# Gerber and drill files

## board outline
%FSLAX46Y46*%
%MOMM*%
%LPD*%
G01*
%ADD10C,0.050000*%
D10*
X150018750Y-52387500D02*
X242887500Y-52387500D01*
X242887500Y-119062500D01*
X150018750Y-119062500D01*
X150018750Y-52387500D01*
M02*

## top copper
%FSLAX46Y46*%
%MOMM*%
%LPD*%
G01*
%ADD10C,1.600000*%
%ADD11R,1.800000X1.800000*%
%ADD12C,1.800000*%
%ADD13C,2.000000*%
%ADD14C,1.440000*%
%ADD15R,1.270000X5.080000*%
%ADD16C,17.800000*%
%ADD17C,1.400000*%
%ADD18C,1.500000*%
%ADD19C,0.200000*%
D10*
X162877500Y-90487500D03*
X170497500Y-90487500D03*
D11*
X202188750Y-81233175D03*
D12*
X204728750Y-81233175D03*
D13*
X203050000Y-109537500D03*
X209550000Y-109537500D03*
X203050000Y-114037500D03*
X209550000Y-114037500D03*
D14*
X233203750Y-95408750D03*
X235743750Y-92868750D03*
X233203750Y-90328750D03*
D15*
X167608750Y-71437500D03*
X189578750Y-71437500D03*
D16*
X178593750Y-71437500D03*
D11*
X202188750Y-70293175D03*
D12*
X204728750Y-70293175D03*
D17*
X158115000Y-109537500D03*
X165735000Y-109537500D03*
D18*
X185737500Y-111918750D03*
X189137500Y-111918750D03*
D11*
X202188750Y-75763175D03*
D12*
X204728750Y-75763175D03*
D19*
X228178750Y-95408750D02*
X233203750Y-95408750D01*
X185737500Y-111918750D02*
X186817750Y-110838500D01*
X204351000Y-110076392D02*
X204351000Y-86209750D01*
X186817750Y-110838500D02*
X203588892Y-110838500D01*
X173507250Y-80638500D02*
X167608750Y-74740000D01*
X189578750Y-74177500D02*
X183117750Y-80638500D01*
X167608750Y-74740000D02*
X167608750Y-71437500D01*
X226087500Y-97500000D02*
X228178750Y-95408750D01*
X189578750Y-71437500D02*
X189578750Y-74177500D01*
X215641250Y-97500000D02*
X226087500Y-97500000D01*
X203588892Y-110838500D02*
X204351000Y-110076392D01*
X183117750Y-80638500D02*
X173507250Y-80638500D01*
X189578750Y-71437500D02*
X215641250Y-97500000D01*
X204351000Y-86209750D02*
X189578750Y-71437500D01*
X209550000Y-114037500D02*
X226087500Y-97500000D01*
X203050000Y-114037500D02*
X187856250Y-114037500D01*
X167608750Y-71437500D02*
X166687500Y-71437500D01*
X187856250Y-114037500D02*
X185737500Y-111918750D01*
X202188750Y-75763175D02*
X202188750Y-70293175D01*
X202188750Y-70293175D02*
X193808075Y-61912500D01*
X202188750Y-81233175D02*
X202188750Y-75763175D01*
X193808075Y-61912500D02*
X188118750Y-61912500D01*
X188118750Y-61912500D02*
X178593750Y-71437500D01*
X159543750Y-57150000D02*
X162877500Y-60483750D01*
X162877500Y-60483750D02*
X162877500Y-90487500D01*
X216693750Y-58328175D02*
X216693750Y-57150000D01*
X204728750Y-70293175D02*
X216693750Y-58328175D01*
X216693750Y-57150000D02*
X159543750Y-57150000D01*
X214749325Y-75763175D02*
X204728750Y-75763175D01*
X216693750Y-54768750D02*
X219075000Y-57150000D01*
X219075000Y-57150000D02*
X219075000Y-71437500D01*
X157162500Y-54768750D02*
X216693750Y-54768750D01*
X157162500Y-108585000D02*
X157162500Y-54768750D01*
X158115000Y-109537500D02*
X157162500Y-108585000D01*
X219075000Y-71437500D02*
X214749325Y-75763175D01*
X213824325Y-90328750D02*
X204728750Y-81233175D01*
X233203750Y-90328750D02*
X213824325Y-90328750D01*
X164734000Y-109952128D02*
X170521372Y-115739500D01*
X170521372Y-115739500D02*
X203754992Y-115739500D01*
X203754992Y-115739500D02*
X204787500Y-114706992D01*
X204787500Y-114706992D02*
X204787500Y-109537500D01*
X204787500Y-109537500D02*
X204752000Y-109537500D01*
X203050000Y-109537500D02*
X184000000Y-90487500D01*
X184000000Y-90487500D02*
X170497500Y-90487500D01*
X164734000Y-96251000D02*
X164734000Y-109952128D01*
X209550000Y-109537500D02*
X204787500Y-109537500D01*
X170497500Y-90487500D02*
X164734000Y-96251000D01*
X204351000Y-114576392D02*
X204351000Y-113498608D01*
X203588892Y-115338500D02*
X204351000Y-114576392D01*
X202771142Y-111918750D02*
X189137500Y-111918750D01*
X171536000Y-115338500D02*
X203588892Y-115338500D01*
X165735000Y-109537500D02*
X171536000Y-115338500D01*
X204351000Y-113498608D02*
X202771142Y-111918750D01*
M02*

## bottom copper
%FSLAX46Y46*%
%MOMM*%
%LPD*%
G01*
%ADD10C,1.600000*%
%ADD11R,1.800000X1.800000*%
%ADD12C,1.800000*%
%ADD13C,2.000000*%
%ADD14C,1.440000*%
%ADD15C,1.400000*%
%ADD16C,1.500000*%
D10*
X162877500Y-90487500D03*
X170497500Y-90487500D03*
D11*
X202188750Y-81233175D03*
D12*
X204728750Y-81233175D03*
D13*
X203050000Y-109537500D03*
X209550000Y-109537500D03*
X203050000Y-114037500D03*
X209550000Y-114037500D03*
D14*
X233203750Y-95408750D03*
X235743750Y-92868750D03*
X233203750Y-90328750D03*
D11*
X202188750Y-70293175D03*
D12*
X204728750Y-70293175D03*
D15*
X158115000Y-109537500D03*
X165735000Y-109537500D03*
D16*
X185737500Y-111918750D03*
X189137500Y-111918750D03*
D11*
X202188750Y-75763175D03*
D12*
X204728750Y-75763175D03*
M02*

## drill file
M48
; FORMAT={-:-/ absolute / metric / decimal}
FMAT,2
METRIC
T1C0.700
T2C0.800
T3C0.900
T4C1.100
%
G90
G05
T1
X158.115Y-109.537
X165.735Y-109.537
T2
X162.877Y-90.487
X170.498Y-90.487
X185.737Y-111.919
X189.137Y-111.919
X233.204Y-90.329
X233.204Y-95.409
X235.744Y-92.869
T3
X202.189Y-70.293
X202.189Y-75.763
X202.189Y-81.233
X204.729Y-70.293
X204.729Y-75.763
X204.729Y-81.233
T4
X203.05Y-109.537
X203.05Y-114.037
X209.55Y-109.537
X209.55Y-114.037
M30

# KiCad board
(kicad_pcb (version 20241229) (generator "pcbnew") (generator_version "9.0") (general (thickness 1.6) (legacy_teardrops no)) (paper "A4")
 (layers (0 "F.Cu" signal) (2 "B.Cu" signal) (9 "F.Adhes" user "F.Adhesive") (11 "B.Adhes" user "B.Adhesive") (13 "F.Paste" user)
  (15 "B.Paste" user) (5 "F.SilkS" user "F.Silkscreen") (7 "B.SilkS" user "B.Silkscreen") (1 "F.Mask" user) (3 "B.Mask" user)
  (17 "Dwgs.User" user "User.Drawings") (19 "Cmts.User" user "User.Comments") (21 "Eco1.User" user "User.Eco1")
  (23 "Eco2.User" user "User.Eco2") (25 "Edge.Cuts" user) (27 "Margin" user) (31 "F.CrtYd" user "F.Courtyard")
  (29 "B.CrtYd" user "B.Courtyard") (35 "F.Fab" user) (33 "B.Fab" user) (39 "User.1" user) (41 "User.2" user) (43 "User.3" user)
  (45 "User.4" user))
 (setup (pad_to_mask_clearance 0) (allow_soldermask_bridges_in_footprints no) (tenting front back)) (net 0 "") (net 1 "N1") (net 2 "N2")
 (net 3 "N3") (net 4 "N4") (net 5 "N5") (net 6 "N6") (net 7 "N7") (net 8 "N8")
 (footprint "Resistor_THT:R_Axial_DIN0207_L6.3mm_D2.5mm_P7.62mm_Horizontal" (layer "F.Cu") (at 162.8775 90.4875)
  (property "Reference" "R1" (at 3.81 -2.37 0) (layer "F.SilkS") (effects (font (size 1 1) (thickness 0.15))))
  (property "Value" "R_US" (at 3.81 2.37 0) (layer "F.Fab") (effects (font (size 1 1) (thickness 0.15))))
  (pad "1" thru_hole circle (at 0 0) (size 1.6 1.6) (drill 0.8) (layers "*.Cu" "*.Mask") (remove_unused_layers no) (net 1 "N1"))
  (pad "2" thru_hole circle (at 7.62 0) (size 1.6 1.6) (drill 0.8) (layers "*.Cu" "*.Mask") (remove_unused_layers no) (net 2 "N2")))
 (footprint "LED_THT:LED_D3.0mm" (layer "F.Cu") (at 202.18875 81.233175)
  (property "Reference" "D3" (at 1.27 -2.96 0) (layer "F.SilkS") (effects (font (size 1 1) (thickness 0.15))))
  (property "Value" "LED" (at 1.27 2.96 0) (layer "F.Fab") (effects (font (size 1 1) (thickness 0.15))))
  (pad "1" thru_hole rect (at 0 0) (size 1.8 1.8) (drill 0.9) (layers "*.Cu" "*.Mask") (remove_unused_layers no) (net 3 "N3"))
  (pad "2" thru_hole circle (at 2.54 0) (size 1.8 1.8) (drill 0.9) (layers "*.Cu" "*.Mask") (remove_unused_layers no) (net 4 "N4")))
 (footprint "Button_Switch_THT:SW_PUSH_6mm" (layer "F.Cu") (at 203.05 109.5375)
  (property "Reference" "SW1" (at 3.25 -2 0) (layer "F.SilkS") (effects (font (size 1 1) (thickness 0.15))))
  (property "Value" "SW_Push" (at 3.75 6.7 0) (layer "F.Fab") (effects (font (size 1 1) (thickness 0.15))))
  (pad "1" thru_hole circle (at 0 0 90) (size 2 2) (drill 1.1) (layers "*.Cu" "*.Mask") (remove_unused_layers no) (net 2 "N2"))
  (pad "1" thru_hole circle (at 6.5 0 90) (size 2 2) (drill 1.1) (layers "*.Cu" "*.Mask") (remove_unused_layers no) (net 2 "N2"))
  (pad "2" thru_hole circle (at 0 4.5 90) (size 2 2) (drill 1.1) (layers "*.Cu" "*.Mask") (remove_unused_layers no) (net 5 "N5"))
  (pad "2" thru_hole circle (at 6.5 4.5 90) (size 2 2) (drill 1.1) (layers "*.Cu" "*.Mask") (remove_unused_layers no) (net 5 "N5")))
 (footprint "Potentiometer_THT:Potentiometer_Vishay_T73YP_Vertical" (layer "F.Cu") (at 233.20375 95.40875)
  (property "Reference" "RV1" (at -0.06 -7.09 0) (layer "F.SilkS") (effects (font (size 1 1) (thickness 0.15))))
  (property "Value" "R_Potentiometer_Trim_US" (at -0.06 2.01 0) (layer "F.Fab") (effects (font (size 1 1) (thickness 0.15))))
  (pad "1" thru_hole circle (at 0 0) (size 1.44 1.44) (drill 0.8) (layers "*.Cu" "*.Mask") (remove_unused_layers no) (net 5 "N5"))
  (pad "2" thru_hole circle (at 2.54 -2.54) (size 1.44 1.44) (drill 0.8) (layers "*.Cu" "*.Mask") (remove_unused_layers no) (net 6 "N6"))
  (pad "3" thru_hole circle (at 0 -5.08) (size 1.44 1.44) (drill 0.8) (layers "*.Cu" "*.Mask") (remove_unused_layers no) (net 4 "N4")))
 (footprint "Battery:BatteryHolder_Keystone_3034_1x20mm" (layer "F.Cu") (at 178.59375 71.4375)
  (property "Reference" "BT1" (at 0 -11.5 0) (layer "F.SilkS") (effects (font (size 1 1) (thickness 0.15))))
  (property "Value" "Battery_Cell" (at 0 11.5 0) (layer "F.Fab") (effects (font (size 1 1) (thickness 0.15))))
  (pad "1" smd rect (at -10.985 0) (size 1.27 5.08) (layers "F.Cu" "F.Mask" "F.Paste") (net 5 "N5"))
  (pad "1" smd rect (at 10.985 0) (size 1.27 5.08) (layers "F.Cu" "F.Mask" "F.Paste") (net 5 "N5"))
  (pad "2" smd circle (at 0 0) (size 17.8 17.8) (layers "F.Cu" "F.Mask") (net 3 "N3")))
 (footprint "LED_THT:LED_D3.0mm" (layer "F.Cu") (at 202.18875 70.293175)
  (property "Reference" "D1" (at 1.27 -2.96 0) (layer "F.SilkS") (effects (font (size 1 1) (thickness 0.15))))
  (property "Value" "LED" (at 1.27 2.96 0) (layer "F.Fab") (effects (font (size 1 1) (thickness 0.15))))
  (pad "1" thru_hole rect (at 0 0) (size 1.8 1.8) (drill 0.9) (layers "*.Cu" "*.Mask") (remove_unused_layers no) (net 3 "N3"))
  (pad "2" thru_hole circle (at 2.54 0) (size 1.8 1.8) (drill 0.9) (layers "*.Cu" "*.Mask") (remove_unused_layers no) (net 1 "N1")))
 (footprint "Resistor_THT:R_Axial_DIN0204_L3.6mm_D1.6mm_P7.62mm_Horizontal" (layer "F.Cu") (at 158.115 109.5375)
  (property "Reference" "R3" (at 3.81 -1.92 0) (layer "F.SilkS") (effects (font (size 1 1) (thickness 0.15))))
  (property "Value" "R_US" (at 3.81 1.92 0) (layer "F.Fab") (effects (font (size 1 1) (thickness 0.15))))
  (pad "1" thru_hole circle (at 0 0) (size 1.4 1.4) (drill 0.7) (layers "*.Cu" "*.Mask") (remove_unused_layers no) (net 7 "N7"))
  (pad "2" thru_hole circle (at 7.62 0) (size 1.4 1.4) (drill 0.7) (layers "*.Cu" "*.Mask") (remove_unused_layers no) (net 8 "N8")))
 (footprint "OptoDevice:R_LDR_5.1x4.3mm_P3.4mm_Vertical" (layer "F.Cu") (at 185.7375 111.91875)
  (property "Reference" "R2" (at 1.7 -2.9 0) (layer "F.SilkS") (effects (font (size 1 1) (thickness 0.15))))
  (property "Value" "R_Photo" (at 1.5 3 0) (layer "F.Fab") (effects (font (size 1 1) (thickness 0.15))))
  (pad "1" thru_hole circle (at 0 0) (size 1.5 1.5) (drill 0.8) (layers "*.Cu" "*.Mask") (remove_unused_layers no) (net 5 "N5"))
  (pad "2" thru_hole circle (at 3.4 0) (size 1.5 1.5) (drill 0.8) (layers "*.Cu" "*.Mask") (remove_unused_layers no) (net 8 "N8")))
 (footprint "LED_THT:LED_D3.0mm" (layer "F.Cu") (at 202.18875 75.763175)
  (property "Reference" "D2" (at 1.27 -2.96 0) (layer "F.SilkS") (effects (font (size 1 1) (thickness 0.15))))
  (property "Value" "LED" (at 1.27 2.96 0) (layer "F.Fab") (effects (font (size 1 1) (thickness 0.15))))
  (pad "1" thru_hole rect (at 0 0) (size 1.8 1.8) (drill 0.9) (layers "*.Cu" "*.Mask") (remove_unused_layers no) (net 3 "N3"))
  (pad "2" thru_hole circle (at 2.54 0) (size 1.8 1.8) (drill 0.9) (layers "*.Cu" "*.Mask") (remove_unused_layers no) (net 7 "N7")))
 (gr_rect (start 150.01875 52.3875) (end 242.8875 119.0625) (stroke (width 0.05) (type default)) (fill no) (layer "Edge.Cuts"))
 (segment (start 228.17875 95.40875) (end 233.20375 95.40875) (width 0.2) (layer "F.Cu") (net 5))
 (segment (start 185.7375 111.91875) (end 186.81775 110.8385) (width 0.2) (layer "F.Cu") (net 5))
 (segment (start 204.351 110.076392) (end 204.351 86.20975) (width 0.2) (layer "F.Cu") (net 5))
 (segment (start 186.81775 110.8385) (end 203.588892 110.8385) (width 0.2) (layer "F.Cu") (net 5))
 (segment (start 173.50725 80.6385) (end 167.60875 74.74) (width 0.2) (layer "F.Cu") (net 5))
 (segment (start 189.57875 74.1775) (end 183.11775 80.6385) (width 0.2) (layer "F.Cu") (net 5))
 (segment (start 167.60875 74.74) (end 167.60875 71.4375) (width 0.2) (layer "F.Cu") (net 5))
 (segment (start 226.0875 97.5) (end 228.17875 95.40875) (width 0.2) (layer "F.Cu") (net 5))
 (segment (start 189.57875 71.4375) (end 189.57875 74.1775) (width 0.2) (layer "F.Cu") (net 5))
 (segment (start 215.64125 97.5) (end 226.0875 97.5) (width 0.2) (layer "F.Cu") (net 5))
 (segment (start 203.588892 110.8385) (end 204.351 110.076392) (width 0.2) (layer "F.Cu") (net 5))
 (segment (start 183.11775 80.6385) (end 173.50725 80.6385) (width 0.2) (layer "F.Cu") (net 5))
 (segment (start 189.57875 71.4375) (end 215.64125 97.5) (width 0.2) (layer "F.Cu") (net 5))
 (segment (start 204.351 86.20975) (end 189.57875 71.4375) (width 0.2) (layer "F.Cu") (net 5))
 (segment (start 209.55 114.0375) (end 226.0875 97.5) (width 0.2) (layer "F.Cu") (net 5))
 (segment (start 203.05 114.0375) (end 187.85625 114.0375) (width 0.2) (layer "F.Cu") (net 5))
 (segment (start 167.60875 71.4375) (end 166.6875 71.4375) (width 0.2) (layer "F.Cu") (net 5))
 (segment (start 187.85625 114.0375) (end 185.7375 111.91875) (width 0.2) (layer "F.Cu") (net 5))
 (segment (start 202.18875 75.763175) (end 202.18875 70.293175) (width 0.2) (layer "F.Cu") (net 3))
 (segment (start 202.18875 70.293175) (end 193.808075 61.9125) (width 0.2) (layer "F.Cu") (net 3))
 (segment (start 202.18875 81.233175) (end 202.18875 75.763175) (width 0.2) (layer "F.Cu") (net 3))
 (segment (start 193.808075 61.9125) (end 188.11875 61.9125) (width 0.2) (layer "F.Cu") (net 3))
 (segment (start 188.11875 61.9125) (end 178.59375 71.4375) (width 0.2) (layer "F.Cu") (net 3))
 (segment (start 159.54375 57.15) (end 162.8775 60.48375) (width 0.2) (layer "F.Cu") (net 1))
 (segment (start 162.8775 60.48375) (end 162.8775 90.4875) (width 0.2) (layer "F.Cu") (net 1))
 (segment (start 216.69375 58.328175) (end 216.69375 57.15) (width 0.2) (layer "F.Cu") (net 1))
 (segment (start 204.72875 70.293175) (end 216.69375 58.328175) (width 0.2) (layer "F.Cu") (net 1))
 (segment (start 216.69375 57.15) (end 159.54375 57.15) (width 0.2) (layer "F.Cu") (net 1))
 (segment (start 214.749325 75.763175) (end 204.72875 75.763175) (width 0.2) (layer "F.Cu") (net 7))
 (segment (start 216.69375 54.76875) (end 219.075 57.15) (width 0.2) (layer "F.Cu") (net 7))
 (segment (start 219.075 57.15) (end 219.075 71.4375) (width 0.2) (layer "F.Cu") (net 7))
 (segment (start 157.1625 54.76875) (end 216.69375 54.76875) (width 0.2) (layer "F.Cu") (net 7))
 (segment (start 157.1625 108.585) (end 157.1625 54.76875) (width 0.2) (layer "F.Cu") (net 7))
 (segment (start 158.115 109.5375) (end 157.1625 108.585) (width 0.2) (layer "F.Cu") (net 7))
 (segment (start 219.075 71.4375) (end 214.749325 75.763175) (width 0.2) (layer "F.Cu") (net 7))
 (segment (start 213.824325 90.32875) (end 204.72875 81.233175) (width 0.2) (layer "F.Cu") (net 4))
 (segment (start 233.20375 90.32875) (end 213.824325 90.32875) (width 0.2) (layer "F.Cu") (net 4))
 (segment (start 164.734 109.952128) (end 170.521372 115.7395) (width 0.2) (layer "F.Cu") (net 2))
 (segment (start 170.521372 115.7395) (end 203.754992 115.7395) (width 0.2) (layer "F.Cu") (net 2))
 (segment (start 203.754992 115.7395) (end 204.7875 114.706992) (width 0.2) (layer "F.Cu") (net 2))
 (segment (start 204.7875 114.706992) (end 204.7875 109.5375) (width 0.2) (layer "F.Cu") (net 2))
 (segment (start 204.7875 109.5375) (end 204.752 109.5375) (width 0.2) (layer "F.Cu") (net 2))
 (segment (start 203.05 109.5375) (end 184 90.4875) (width 0.2) (layer "F.Cu") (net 2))
 (segment (start 184 90.4875) (end 170.4975 90.4875) (width 0.2) (layer "F.Cu") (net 2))
 (segment (start 164.734 96.251) (end 164.734 109.952128) (width 0.2) (layer "F.Cu") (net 2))
 (segment (start 209.55 109.5375) (end 204.7875 109.5375) (width 0.2) (layer "F.Cu") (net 2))
 (segment (start 170.4975 90.4875) (end 164.734 96.251) (width 0.2) (layer "F.Cu") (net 2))
 (segment (start 204.351 114.576392) (end 204.351 113.498608) (width 0.2) (layer "F.Cu") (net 8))
 (segment (start 203.588892 115.3385) (end 204.351 114.576392) (width 0.2) (layer "F.Cu") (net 8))
 (segment (start 202.771142 111.91875) (end 189.1375 111.91875) (width 0.2) (layer "F.Cu") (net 8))
 (segment (start 171.536 115.3385) (end 203.588892 115.3385) (width 0.2) (layer "F.Cu") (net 8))
 (segment (start 165.735 109.5375) (end 171.536 115.3385) (width 0.2) (layer "F.Cu") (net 8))
 (segment (start 204.351 113.498608) (end 202.771142 111.91875) (width 0.2) (layer "F.Cu") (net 8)))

